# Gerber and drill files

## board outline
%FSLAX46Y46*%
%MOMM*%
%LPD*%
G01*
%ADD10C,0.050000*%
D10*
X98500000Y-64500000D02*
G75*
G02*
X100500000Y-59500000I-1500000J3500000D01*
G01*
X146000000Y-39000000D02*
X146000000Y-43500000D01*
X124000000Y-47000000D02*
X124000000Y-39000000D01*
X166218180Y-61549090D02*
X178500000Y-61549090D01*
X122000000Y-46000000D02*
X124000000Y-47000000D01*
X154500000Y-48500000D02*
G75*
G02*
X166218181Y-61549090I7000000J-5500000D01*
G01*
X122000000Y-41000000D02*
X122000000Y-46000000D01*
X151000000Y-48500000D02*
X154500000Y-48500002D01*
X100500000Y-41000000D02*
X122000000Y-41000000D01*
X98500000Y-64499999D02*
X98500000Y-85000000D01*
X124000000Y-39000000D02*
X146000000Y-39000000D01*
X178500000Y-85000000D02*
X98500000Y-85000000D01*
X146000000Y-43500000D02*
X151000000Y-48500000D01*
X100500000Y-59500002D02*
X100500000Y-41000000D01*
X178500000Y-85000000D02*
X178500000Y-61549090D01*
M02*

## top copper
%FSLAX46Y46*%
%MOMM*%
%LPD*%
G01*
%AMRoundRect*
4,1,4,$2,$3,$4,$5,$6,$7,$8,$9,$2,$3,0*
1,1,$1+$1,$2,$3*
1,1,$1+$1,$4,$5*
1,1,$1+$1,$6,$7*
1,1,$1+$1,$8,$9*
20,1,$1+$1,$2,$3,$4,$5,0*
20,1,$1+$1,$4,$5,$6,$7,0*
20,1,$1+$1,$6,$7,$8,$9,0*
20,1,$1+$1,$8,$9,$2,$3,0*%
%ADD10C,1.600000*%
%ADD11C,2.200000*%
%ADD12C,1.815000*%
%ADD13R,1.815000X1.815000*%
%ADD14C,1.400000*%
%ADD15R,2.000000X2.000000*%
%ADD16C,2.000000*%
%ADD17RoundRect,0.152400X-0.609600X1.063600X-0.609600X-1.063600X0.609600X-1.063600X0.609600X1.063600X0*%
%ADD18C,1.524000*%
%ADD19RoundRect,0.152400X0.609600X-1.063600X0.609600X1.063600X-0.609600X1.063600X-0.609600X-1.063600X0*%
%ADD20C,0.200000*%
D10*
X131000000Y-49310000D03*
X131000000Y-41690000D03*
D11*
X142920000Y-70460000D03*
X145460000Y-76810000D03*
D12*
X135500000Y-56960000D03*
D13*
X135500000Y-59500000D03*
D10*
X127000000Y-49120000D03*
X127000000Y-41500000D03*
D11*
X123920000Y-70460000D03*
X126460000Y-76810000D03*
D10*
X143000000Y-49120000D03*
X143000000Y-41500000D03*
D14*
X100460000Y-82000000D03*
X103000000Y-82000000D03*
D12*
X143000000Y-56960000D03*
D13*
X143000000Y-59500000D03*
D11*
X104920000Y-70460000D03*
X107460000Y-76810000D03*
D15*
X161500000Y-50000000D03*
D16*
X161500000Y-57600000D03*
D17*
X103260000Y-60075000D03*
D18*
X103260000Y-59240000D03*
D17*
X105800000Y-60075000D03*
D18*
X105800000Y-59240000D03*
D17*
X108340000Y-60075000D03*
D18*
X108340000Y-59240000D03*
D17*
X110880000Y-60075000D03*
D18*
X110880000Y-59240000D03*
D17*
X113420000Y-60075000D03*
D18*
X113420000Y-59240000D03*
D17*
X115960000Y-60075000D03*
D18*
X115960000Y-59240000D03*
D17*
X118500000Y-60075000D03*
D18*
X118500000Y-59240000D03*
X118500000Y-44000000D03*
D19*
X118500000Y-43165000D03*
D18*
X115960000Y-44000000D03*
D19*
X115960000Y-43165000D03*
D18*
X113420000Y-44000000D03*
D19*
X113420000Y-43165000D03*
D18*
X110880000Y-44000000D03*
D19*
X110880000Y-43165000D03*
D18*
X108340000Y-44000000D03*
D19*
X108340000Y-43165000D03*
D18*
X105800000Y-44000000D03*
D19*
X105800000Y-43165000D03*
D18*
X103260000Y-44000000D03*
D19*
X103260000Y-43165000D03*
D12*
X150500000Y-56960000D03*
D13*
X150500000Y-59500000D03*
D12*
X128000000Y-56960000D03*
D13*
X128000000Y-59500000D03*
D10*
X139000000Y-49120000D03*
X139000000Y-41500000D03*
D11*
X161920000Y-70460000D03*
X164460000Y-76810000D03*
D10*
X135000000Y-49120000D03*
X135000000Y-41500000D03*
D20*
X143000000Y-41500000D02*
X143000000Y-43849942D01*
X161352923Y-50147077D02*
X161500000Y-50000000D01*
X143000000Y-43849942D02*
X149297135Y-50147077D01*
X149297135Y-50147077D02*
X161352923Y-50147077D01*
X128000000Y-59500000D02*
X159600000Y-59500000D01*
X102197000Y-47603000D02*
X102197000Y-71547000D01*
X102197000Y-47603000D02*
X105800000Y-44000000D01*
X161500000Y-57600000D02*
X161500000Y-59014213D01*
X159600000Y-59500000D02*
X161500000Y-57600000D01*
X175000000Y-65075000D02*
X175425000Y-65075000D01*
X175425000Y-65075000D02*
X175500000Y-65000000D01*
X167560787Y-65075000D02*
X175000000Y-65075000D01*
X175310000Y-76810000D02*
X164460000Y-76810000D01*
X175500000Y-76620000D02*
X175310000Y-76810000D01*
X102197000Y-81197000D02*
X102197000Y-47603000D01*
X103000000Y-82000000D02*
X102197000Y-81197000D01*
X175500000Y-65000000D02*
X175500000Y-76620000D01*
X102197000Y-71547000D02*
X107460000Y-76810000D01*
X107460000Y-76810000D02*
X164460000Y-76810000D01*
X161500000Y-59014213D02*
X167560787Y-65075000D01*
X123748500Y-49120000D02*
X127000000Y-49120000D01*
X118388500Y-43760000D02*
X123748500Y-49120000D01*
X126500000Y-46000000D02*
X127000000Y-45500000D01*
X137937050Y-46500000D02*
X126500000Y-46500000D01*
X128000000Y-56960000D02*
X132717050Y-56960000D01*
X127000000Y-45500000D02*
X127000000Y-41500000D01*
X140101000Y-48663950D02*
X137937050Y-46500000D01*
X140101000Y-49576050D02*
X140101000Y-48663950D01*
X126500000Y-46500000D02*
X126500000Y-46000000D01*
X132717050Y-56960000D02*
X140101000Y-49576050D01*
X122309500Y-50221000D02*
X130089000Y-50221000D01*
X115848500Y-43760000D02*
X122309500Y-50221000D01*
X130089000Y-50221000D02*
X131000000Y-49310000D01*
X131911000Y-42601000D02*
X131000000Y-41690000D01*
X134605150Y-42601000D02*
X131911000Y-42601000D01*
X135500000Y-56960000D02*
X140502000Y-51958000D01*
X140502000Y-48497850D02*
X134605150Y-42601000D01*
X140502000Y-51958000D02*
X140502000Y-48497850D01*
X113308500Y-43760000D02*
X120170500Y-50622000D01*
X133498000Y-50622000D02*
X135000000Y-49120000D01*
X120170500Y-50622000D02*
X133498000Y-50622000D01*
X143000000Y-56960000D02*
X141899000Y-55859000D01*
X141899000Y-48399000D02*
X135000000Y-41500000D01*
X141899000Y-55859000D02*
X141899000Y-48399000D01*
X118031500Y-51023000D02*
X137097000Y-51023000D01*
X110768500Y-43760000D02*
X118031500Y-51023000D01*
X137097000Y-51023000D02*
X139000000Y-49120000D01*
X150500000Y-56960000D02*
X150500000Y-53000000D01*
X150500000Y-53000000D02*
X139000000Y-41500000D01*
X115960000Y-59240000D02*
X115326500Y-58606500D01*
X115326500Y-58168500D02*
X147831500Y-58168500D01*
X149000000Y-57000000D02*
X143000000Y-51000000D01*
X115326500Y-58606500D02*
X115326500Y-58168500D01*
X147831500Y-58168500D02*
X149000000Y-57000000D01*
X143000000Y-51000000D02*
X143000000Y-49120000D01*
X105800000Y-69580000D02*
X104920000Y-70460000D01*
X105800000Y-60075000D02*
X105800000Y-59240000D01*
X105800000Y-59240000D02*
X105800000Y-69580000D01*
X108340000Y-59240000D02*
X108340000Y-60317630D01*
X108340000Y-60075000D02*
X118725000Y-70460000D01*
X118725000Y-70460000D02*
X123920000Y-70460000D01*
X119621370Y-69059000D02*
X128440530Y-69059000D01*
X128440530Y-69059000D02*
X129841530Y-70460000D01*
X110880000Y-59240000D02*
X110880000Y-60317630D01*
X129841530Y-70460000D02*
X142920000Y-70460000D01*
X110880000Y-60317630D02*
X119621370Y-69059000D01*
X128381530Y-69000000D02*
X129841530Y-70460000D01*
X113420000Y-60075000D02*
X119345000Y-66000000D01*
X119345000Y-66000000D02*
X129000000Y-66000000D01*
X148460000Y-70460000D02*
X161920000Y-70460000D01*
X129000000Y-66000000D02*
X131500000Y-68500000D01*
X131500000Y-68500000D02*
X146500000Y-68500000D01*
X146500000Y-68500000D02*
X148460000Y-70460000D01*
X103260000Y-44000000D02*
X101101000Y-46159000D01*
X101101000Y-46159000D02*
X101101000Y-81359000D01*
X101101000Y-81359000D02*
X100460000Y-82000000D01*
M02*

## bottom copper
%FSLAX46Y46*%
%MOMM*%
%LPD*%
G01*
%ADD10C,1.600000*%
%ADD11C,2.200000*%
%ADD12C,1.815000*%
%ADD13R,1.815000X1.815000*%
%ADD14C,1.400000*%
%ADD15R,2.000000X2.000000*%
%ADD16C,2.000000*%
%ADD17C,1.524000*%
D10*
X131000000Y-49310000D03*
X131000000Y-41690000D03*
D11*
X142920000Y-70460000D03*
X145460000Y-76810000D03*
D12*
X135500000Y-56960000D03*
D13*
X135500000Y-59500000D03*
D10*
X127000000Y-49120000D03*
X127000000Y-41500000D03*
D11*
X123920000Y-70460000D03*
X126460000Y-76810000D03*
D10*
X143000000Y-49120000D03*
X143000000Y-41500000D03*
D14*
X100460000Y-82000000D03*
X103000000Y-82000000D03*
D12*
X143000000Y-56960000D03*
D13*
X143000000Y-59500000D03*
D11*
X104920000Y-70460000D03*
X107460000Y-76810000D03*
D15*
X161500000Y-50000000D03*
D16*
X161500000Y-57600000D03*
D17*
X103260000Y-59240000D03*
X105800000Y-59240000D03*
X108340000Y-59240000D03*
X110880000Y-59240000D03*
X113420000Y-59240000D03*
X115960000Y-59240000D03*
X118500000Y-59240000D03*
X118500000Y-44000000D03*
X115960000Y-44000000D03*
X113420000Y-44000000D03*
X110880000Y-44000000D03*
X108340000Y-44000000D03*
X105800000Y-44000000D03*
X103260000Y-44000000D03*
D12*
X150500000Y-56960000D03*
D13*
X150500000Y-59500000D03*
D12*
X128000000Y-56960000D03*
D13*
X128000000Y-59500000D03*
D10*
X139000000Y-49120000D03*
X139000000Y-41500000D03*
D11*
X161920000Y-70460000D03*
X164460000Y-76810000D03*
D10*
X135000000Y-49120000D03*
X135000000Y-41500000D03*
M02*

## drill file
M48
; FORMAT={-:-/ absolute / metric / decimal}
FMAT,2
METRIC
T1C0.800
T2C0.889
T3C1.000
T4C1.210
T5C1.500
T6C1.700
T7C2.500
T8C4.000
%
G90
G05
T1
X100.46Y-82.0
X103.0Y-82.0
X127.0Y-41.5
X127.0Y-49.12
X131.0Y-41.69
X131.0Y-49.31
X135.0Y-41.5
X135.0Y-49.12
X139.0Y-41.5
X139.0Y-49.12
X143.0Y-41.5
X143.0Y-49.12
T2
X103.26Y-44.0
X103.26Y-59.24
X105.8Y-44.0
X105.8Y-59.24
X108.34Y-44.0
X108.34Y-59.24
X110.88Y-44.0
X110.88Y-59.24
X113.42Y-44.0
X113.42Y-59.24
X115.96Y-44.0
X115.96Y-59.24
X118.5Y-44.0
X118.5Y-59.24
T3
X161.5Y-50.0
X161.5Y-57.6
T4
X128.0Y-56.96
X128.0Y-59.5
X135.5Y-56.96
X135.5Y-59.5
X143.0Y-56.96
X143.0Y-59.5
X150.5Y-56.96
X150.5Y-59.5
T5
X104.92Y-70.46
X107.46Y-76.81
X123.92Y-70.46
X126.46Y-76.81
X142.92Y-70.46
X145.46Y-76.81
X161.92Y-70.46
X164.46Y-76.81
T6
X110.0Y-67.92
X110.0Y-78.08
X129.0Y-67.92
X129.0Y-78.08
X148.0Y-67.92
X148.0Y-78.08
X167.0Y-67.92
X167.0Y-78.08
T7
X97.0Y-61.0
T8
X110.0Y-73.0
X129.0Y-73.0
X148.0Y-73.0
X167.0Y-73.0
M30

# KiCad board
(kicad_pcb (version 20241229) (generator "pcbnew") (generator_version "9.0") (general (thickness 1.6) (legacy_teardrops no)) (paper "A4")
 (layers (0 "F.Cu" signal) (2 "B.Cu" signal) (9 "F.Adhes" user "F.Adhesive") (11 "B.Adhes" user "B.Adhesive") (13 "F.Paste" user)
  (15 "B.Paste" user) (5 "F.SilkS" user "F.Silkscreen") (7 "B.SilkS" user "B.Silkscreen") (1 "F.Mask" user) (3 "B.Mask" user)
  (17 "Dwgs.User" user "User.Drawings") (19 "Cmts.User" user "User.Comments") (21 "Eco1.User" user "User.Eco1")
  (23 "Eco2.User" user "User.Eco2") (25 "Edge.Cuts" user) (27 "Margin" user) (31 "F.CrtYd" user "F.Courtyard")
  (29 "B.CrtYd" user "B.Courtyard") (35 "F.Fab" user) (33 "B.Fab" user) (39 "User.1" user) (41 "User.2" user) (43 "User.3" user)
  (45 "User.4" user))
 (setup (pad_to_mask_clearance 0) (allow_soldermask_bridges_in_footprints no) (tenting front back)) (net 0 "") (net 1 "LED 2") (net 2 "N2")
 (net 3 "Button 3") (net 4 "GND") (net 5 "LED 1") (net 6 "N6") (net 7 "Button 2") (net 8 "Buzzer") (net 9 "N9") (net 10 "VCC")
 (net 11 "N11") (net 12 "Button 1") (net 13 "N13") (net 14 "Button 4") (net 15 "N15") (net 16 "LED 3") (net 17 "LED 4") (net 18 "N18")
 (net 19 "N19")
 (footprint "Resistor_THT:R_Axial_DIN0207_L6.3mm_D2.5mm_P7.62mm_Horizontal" (layer "F.Cu") (at 131 49.31 90)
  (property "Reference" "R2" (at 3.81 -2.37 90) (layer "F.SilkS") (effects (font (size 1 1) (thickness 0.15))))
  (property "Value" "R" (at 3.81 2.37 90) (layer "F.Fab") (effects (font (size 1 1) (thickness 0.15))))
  (pad "1" thru_hole circle (at 0 0 90) (size 1.6 1.6) (drill 0.8) (layers "*.Cu" "*.Mask") (remove_unused_layers no) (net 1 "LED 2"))
  (pad "2" thru_hole circle (at 7.62 0 90) (size 1.6 1.6) (drill 0.8) (layers "*.Cu" "*.Mask") (remove_unused_layers no) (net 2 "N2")))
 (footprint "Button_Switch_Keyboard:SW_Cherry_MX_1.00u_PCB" (layer "F.Cu") (at 142.92 70.46 90)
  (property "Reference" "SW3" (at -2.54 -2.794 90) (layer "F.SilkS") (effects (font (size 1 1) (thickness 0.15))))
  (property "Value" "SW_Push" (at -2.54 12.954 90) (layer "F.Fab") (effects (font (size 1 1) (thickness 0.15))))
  (pad "" np_thru_hole circle (at -7.62 5.08 90) (size 1.7 1.7) (drill 1.7) (layers "*.Cu" "*.Mask"))
  (pad "" np_thru_hole circle (at -2.54 5.08 90) (size 4 4) (drill 4) (layers "*.Cu" "*.Mask"))
  (pad "" np_thru_hole circle (at 2.54 5.08 90) (size 1.7 1.7) (drill 1.7) (layers "*.Cu" "*.Mask"))
  (pad "1" thru_hole circle (at 0 0 90) (size 2.2 2.2) (drill 1.5) (layers "*.Cu" "*.Mask") (remove_unused_layers no) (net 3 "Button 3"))
  (pad "2" thru_hole circle (at -6.35 2.54 90) (size 2.2 2.2) (drill 1.5) (layers "*.Cu" "*.Mask") (remove_unused_layers no) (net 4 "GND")))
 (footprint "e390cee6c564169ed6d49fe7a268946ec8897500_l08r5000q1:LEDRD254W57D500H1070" (layer "F.Cu") (at 135.5 58.23 90)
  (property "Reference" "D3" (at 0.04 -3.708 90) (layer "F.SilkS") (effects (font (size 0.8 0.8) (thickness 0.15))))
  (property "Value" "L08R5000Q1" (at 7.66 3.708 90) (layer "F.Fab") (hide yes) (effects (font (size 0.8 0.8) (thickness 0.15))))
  (pad "A" thru_hole circle (at 1.27 0 90) (size 1.815 1.815) (drill 1.21) (layers "*.Cu" "*.Mask") (remove_unused_layers no) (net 2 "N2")
   (solder_mask_margin 0.102))
  (pad "C" thru_hole rect (at -1.27 0 90) (size 1.815 1.815) (drill 1.21) (layers "*.Cu" "*.Mask") (remove_unused_layers no) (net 4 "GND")
   (solder_mask_margin 0.102)))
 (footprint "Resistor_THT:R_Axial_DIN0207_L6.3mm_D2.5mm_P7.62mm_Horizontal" (layer "F.Cu") (at 127 49.12 90)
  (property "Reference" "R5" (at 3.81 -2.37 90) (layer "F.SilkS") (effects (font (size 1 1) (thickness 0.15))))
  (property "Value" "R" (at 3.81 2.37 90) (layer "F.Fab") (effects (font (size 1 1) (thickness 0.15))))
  (pad "1" thru_hole circle (at 0 0 90) (size 1.6 1.6) (drill 0.8) (layers "*.Cu" "*.Mask") (remove_unused_layers no) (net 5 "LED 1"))
  (pad "2" thru_hole circle (at 7.62 0 90) (size 1.6 1.6) (drill 0.8) (layers "*.Cu" "*.Mask") (remove_unused_layers no) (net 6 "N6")))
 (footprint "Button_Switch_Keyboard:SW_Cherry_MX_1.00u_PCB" (layer "F.Cu") (at 123.92 70.46 90)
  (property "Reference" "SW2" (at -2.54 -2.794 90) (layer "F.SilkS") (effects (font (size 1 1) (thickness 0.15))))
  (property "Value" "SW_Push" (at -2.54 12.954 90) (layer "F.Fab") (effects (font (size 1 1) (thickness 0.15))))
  (pad "" np_thru_hole circle (at -7.62 5.08 90) (size 1.7 1.7) (drill 1.7) (layers "*.Cu" "*.Mask"))
  (pad "" np_thru_hole circle (at -2.54 5.08 90) (size 4 4) (drill 4) (layers "*.Cu" "*.Mask"))
  (pad "" np_thru_hole circle (at 2.54 5.08 90) (size 1.7 1.7) (drill 1.7) (layers "*.Cu" "*.Mask"))
  (pad "1" thru_hole circle (at 0 0 90) (size 2.2 2.2) (drill 1.5) (layers "*.Cu" "*.Mask") (remove_unused_layers no) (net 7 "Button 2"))
  (pad "2" thru_hole circle (at -6.35 2.54 90) (size 2.2 2.2) (drill 1.5) (layers "*.Cu" "*.Mask") (remove_unused_layers no) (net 4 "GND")))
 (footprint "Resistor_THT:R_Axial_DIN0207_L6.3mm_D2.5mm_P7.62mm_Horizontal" (layer "F.Cu") (at 143 49.12 90)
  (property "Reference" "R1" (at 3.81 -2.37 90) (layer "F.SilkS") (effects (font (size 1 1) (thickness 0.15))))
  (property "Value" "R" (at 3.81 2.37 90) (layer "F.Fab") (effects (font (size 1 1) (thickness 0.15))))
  (pad "1" thru_hole circle (at 0 0 90) (size 1.6 1.6) (drill 0.8) (layers "*.Cu" "*.Mask") (remove_unused_layers no) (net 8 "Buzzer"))
  (pad "2" thru_hole circle (at 7.62 0 90) (size 1.6 1.6) (drill 0.8) (layers "*.Cu" "*.Mask") (remove_unused_layers no) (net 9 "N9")))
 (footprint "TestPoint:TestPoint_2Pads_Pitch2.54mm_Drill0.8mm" (layer "F.Cu") (at 100.46 82)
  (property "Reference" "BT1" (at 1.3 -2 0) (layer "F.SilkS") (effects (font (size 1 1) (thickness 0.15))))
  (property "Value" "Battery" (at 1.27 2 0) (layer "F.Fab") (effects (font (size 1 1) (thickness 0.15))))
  (pad "1" thru_hole circle (at 0 0) (size 1.4 1.4) (drill 0.8) (layers "*.Cu" "*.Mask") (remove_unused_layers no) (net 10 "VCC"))
  (pad "2" thru_hole circle (at 2.54 0) (size 1.4 1.4) (drill 0.8) (layers "*.Cu" "*.Mask") (remove_unused_layers no) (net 4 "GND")))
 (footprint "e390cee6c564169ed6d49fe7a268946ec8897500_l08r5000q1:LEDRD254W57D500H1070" (layer "F.Cu") (at 143 58.23 90)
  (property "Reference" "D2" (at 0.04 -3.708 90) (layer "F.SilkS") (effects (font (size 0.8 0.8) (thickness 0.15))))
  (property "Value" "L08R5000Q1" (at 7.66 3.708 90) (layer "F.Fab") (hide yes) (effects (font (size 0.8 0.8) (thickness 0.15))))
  (pad "A" thru_hole circle (at 1.27 0 90) (size 1.815 1.815) (drill 1.21) (layers "*.Cu" "*.Mask") (remove_unused_layers no) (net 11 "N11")
   (solder_mask_margin 0.102))
  (pad "C" thru_hole rect (at -1.27 0 90) (size 1.815 1.815) (drill 1.21) (layers "*.Cu" "*.Mask") (remove_unused_layers no) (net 4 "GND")
   (solder_mask_margin 0.102)))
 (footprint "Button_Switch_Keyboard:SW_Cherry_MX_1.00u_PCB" (layer "F.Cu") (at 104.92 70.46 90)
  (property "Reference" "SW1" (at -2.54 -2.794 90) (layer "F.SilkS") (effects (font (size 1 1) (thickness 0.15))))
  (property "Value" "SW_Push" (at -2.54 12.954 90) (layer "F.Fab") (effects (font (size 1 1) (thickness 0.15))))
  (pad "" np_thru_hole circle (at -7.62 5.08 90) (size 1.7 1.7) (drill 1.7) (layers "*.Cu" "*.Mask"))
  (pad "" np_thru_hole circle (at -2.54 5.08 90) (size 4 4) (drill 4) (layers "*.Cu" "*.Mask"))
  (pad "" np_thru_hole circle (at 2.54 5.08 90) (size 1.7 1.7) (drill 1.7) (layers "*.Cu" "*.Mask"))
  (pad "1" thru_hole circle (at 0 0 90) (size 2.2 2.2) (drill 1.5) (layers "*.Cu" "*.Mask") (remove_unused_layers no) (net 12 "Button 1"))
  (pad "2" thru_hole circle (at -6.35 2.54 90) (size 2.2 2.2) (drill 1.5) (layers "*.Cu" "*.Mask") (remove_unused_layers no) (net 4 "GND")))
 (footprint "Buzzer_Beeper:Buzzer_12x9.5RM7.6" (layer "F.Cu") (at 161.5 50 -90)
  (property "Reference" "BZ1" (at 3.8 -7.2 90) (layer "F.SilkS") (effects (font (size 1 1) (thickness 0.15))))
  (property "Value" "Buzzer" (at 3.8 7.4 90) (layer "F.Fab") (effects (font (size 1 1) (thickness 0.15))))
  (pad "1" thru_hole rect (at 0 0 270) (size 2 2) (drill 1) (layers "*.Cu" "*.Mask") (remove_unused_layers no) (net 9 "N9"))
  (pad "2" thru_hole circle (at 7.6 0 270) (size 2 2) (drill 1) (layers "*.Cu" "*.Mask") (remove_unused_layers no) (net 4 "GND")))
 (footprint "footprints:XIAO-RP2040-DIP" (layer "F.Cu") (at 110.88 51.62 90)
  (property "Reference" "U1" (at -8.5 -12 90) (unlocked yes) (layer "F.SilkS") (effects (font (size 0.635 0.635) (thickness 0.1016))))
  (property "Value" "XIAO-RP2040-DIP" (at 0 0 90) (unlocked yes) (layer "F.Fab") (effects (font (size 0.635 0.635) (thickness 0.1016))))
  (pad "1" smd roundrect (at -8.455 -7.62 270) (size 2.432 1.524) (layers "F.Cu" "F.Mask") (roundrect_rratio 0.1) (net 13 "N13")
   (thermal_bridge_angle 45))
  (pad "1" thru_hole circle (at -7.62 -7.62 270) (size 1.524 1.524) (drill 0.889) (layers "*.Cu" "*.Mask") (remove_unused_layers no)
   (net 13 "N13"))
  (pad "2" smd roundrect (at -8.455 -5.08 270) (size 2.432 1.524) (layers "F.Cu" "F.Mask") (roundrect_rratio 0.1) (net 12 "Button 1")
   (thermal_bridge_angle 45))
  (pad "2" thru_hole circle (at -7.62 -5.08 270) (size 1.524 1.524) (drill 0.889) (layers "*.Cu" "*.Mask") (remove_unused_layers no)
   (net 12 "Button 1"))
  (pad "3" smd roundrect (at -8.455 -2.54 270) (size 2.432 1.524) (layers "F.Cu" "F.Mask") (roundrect_rratio 0.1) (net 7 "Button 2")
   (thermal_bridge_angle 45))
  (pad "3" thru_hole circle (at -7.62 -2.54 270) (size 1.524 1.524) (drill 0.889) (layers "*.Cu" "*.Mask") (remove_unused_layers no)
   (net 7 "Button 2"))
  (pad "4" smd roundrect (at -8.455 0 270) (size 2.432 1.524) (layers "F.Cu" "F.Mask") (roundrect_rratio 0.1) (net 3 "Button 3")
   (thermal_bridge_angle 45))
  (pad "4" thru_hole circle (at -7.62 0 270) (size 1.524 1.524) (drill 0.889) (layers "*.Cu" "*.Mask") (remove_unused_layers no)
   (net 3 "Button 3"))
  (pad "5" smd roundrect (at -8.455 2.54 270) (size 2.432 1.524) (layers "F.Cu" "F.Mask") (roundrect_rratio 0.1) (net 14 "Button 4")
   (thermal_bridge_angle 45))
  (pad "5" thru_hole circle (at -7.62 2.54 270) (size 1.524 1.524) (drill 0.889) (layers "*.Cu" "*.Mask") (remove_unused_layers no)
   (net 14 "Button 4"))
  (pad "6" smd roundrect (at -8.455 5.08 270) (size 2.432 1.524) (layers "F.Cu" "F.Mask") (roundrect_rratio 0.1) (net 8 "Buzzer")
   (thermal_bridge_angle 45))
  (pad "6" thru_hole circle (at -7.62 5.08 270) (size 1.524 1.524) (drill 0.889) (layers "*.Cu" "*.Mask") (remove_unused_layers no)
   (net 8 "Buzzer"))
  (pad "7" smd roundrect (at -8.455 7.62 270) (size 2.432 1.524) (layers "F.Cu" "F.Mask") (roundrect_rratio 0.1) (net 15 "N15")
   (thermal_bridge_angle 45))
  (pad "7" thru_hole circle (at -7.62 7.62 270) (size 1.524 1.524) (drill 0.889) (layers "*.Cu" "*.Mask") (remove_unused_layers no)
   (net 15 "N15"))
  (pad "8" thru_hole circle (at 7.62 7.62 90) (size 1.524 1.524) (drill 0.889) (layers "*.Cu" "*.Mask") (remove_unused_layers no)
   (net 5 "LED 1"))
  (pad "8" smd roundrect (at 8.455 7.62 90) (size 2.432 1.524) (layers "F.Cu" "F.Mask") (roundrect_rratio 0.1) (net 5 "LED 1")
   (thermal_bridge_angle 45))
  (pad "9" thru_hole circle (at 7.62 5.08 90) (size 1.524 1.524) (drill 0.889) (layers "*.Cu" "*.Mask") (remove_unused_layers no)
   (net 1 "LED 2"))
  (pad "9" smd roundrect (at 8.455 5.08 90) (size 2.432 1.524) (layers "F.Cu" "F.Mask") (roundrect_rratio 0.1) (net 1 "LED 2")
   (thermal_bridge_angle 45))
  (pad "10" thru_hole circle (at 7.62 2.54 90) (size 1.524 1.524) (drill 0.889) (layers "*.Cu" "*.Mask") (remove_unused_layers no)
   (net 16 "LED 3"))
  (pad "10" smd roundrect (at 8.455 2.54 90) (size 2.432 1.524) (layers "F.Cu" "F.Mask") (roundrect_rratio 0.1) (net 16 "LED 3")
   (thermal_bridge_angle 45))
  (pad "11" thru_hole circle (at 7.62 0 90) (size 1.524 1.524) (drill 0.889) (layers "*.Cu" "*.Mask") (remove_unused_layers no)
   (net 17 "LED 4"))
  (pad "11" smd roundrect (at 8.455 0 90) (size 2.432 1.524) (layers "F.Cu" "F.Mask") (roundrect_rratio 0.1) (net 17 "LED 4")
   (thermal_bridge_angle 45))
  (pad "12" thru_hole circle (at 7.62 -2.54 90) (size 1.524 1.524) (drill 0.889) (layers "*.Cu" "*.Mask") (remove_unused_layers no)
   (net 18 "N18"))
  (pad "12" smd roundrect (at 8.455 -2.54 90) (size 2.432 1.524) (layers "F.Cu" "F.Mask") (roundrect_rratio 0.1) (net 18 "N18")
   (thermal_bridge_angle 45))
  (pad "13" thru_hole circle (at 7.62 -5.08 90) (size 1.524 1.524) (drill 0.889) (layers "*.Cu" "*.Mask") (remove_unused_layers no)
   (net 4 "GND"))
  (pad "13" smd roundrect (at 8.455 -5.08 90) (size 2.432 1.524) (layers "F.Cu" "F.Mask") (roundrect_rratio 0.1) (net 4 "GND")
   (thermal_bridge_angle 45))
  (pad "14" thru_hole circle (at 7.62 -7.62 90) (size 1.524 1.524) (drill 0.889) (layers "*.Cu" "*.Mask") (remove_unused_layers no)
   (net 10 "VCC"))
  (pad "14" smd roundrect (at 8.455 -7.62 90) (size 2.432 1.524) (layers "F.Cu" "F.Mask") (roundrect_rratio 0.1) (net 10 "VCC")
   (thermal_bridge_angle 45)))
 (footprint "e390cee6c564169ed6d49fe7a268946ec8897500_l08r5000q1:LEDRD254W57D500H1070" (layer "F.Cu") (at 150.5 58.23 90)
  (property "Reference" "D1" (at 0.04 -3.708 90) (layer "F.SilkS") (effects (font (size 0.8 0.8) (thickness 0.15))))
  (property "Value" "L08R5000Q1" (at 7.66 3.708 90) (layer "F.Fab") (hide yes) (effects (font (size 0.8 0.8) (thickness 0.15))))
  (pad "A" thru_hole circle (at 1.27 0 90) (size 1.815 1.815) (drill 1.21) (layers "*.Cu" "*.Mask") (remove_unused_layers no) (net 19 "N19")
   (solder_mask_margin 0.102))
  (pad "C" thru_hole rect (at -1.27 0 90) (size 1.815 1.815) (drill 1.21) (layers "*.Cu" "*.Mask") (remove_unused_layers no) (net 4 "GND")
   (solder_mask_margin 0.102)))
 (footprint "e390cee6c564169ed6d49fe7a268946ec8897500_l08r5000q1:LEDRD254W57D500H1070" (layer "F.Cu") (at 128 58.23 90)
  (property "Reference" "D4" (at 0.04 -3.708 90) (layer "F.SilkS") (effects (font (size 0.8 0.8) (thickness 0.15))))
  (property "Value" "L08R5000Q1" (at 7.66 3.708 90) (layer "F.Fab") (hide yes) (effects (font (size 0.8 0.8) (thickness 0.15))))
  (pad "A" thru_hole circle (at 1.27 0 90) (size 1.815 1.815) (drill 1.21) (layers "*.Cu" "*.Mask") (remove_unused_layers no) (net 6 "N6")
   (solder_mask_margin 0.102))
  (pad "C" thru_hole rect (at -1.27 0 90) (size 1.815 1.815) (drill 1.21) (layers "*.Cu" "*.Mask") (remove_unused_layers no) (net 4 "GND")
   (solder_mask_margin 0.102)))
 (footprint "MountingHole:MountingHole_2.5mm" (layer "F.Cu") (at 97 61)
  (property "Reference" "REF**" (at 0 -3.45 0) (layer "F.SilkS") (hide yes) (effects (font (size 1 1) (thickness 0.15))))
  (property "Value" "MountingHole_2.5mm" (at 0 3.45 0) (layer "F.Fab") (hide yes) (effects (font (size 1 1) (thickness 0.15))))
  (pad "" np_thru_hole circle (at 0 0) (size 2.5 2.5) (drill 2.5) (layers "*.Cu" "*.Mask")))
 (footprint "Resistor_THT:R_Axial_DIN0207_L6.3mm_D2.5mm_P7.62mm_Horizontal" (layer "F.Cu") (at 139 49.12 90)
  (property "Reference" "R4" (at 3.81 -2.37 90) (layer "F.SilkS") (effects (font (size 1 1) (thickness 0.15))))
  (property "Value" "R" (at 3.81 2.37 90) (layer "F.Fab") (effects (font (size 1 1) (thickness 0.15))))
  (pad "1" thru_hole circle (at 0 0 90) (size 1.6 1.6) (drill 0.8) (layers "*.Cu" "*.Mask") (remove_unused_layers no) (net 17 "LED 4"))
  (pad "2" thru_hole circle (at 7.62 0 90) (size 1.6 1.6) (drill 0.8) (layers "*.Cu" "*.Mask") (remove_unused_layers no) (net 19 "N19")))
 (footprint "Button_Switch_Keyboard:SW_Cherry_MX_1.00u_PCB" (layer "F.Cu") (at 161.92 70.46 90)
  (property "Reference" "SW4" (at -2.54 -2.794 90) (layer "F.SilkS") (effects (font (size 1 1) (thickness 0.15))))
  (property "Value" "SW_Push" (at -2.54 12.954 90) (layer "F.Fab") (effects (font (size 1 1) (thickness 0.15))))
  (pad "" np_thru_hole circle (at -7.62 5.08 90) (size 1.7 1.7) (drill 1.7) (layers "*.Cu" "*.Mask"))
  (pad "" np_thru_hole circle (at -2.54 5.08 90) (size 4 4) (drill 4) (layers "*.Cu" "*.Mask"))
  (pad "" np_thru_hole circle (at 2.54 5.08 90) (size 1.7 1.7) (drill 1.7) (layers "*.Cu" "*.Mask"))
  (pad "1" thru_hole circle (at 0 0 90) (size 2.2 2.2) (drill 1.5) (layers "*.Cu" "*.Mask") (remove_unused_layers no) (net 14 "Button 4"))
  (pad "2" thru_hole circle (at -6.35 2.54 90) (size 2.2 2.2) (drill 1.5) (layers "*.Cu" "*.Mask") (remove_unused_layers no) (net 4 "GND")))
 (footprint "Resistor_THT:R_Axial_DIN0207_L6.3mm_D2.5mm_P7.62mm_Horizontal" (layer "F.Cu") (at 135 49.12 90)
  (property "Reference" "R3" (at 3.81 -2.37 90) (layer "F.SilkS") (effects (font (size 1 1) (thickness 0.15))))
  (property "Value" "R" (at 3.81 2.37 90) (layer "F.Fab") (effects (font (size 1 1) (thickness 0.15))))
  (pad "1" thru_hole circle (at 0 0 90) (size 1.6 1.6) (drill 0.8) (layers "*.Cu" "*.Mask") (remove_unused_layers no) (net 16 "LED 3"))
  (pad "2" thru_hole circle (at 7.62 0 90) (size 1.6 1.6) (drill 0.8) (layers "*.Cu" "*.Mask") (remove_unused_layers no) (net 11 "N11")))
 (gr_arc (start 98.5 64.5) (mid 93.464466 59.585786) (end 100.5 59.5) (stroke (width 0.05) (type default)) (layer "Edge.Cuts"))
 (gr_line (start 146 39) (end 146 43.5) (stroke (width 0.05) (type default)) (layer "Edge.Cuts"))
 (gr_line (start 124 47) (end 124 39) (stroke (width 0.05) (type default)) (layer "Edge.Cuts"))
 (gr_line (start 166.21818 61.54909) (end 178.5 61.54909) (stroke (width 0.05) (type default)) (layer "Edge.Cuts"))
 (gr_line (start 122 46) (end 124 47) (stroke (width 0.05) (type default)) (layer "Edge.Cuts"))
 (gr_arc (start 154.5 48.5) (mid 168.123546 48.052006) (end 166.218181 61.54909) (stroke (width 0.05) (type default)) (layer "Edge.Cuts"))
 (gr_line (start 122 41) (end 122 46) (stroke (width 0.05) (type default)) (layer "Edge.Cuts"))
 (gr_line (start 151 48.5) (end 154.5 48.500002) (stroke (width 0.05) (type default)) (layer "Edge.Cuts"))
 (gr_line (start 100.5 41) (end 122 41) (stroke (width 0.05) (type default)) (layer "Edge.Cuts"))
 (gr_line (start 98.5 64.499999) (end 98.5 85) (stroke (width 0.05) (type default)) (layer "Edge.Cuts"))
 (gr_line (start 124 39) (end 146 39) (stroke (width 0.05) (type default)) (layer "Edge.Cuts"))
 (gr_line (start 178.5 85) (end 98.5 85) (stroke (width 0.05) (type default)) (layer "Edge.Cuts"))
 (gr_line (start 146 43.5) (end 151 48.5) (stroke (width 0.05) (type default)) (layer "Edge.Cuts"))
 (gr_line (start 100.5 59.500002) (end 100.5 41) (stroke (width 0.05) (type default)) (layer "Edge.Cuts"))
 (gr_line (start 178.5 85) (end 178.5 61.54909) (stroke (width 0.05) (type default)) (layer "Edge.Cuts"))
 (segment (start 143 41.5) (end 143 43.849942) (width 0.2) (layer "F.Cu") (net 9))
 (segment (start 161.352923 50.147077) (end 161.5 50) (width 0.2) (layer "F.Cu") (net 9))
 (segment (start 143 43.849942) (end 149.297135 50.147077) (width 0.2) (layer "F.Cu") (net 9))
 (segment (start 149.297135 50.147077) (end 161.352923 50.147077) (width 0.2) (layer "F.Cu") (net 9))
 (segment (start 128 59.5) (end 159.6 59.5) (width 0.2) (layer "F.Cu") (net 4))
 (segment (start 102.197 47.603) (end 102.197 71.547) (width 0.2) (layer "F.Cu") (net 4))
 (segment (start 102.197 47.603) (end 105.8 44) (width 0.2) (layer "F.Cu") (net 4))
 (segment (start 161.5 57.6) (end 161.5 59.014213) (width 0.2) (layer "F.Cu") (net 4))
 (segment (start 159.6 59.5) (end 161.5 57.6) (width 0.2) (layer "F.Cu") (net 4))
 (segment (start 175 65.075) (end 175.425 65.075) (width 0.2) (layer "F.Cu") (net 4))
 (segment (start 175.425 65.075) (end 175.5 65) (width 0.2) (layer "F.Cu") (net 4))
 (segment (start 167.560787 65.075) (end 175 65.075) (width 0.2) (layer "F.Cu") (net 4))
 (segment (start 175.31 76.81) (end 164.46 76.81) (width 0.2) (layer "F.Cu") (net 4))
 (segment (start 175.5 76.62) (end 175.31 76.81) (width 0.2) (layer "F.Cu") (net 4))
 (segment (start 102.197 81.197) (end 102.197 47.603) (width 0.2) (layer "F.Cu") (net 4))
 (segment (start 103 82) (end 102.197 81.197) (width 0.2) (layer "F.Cu") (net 4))
 (segment (start 175.5 65) (end 175.5 76.62) (width 0.2) (layer "F.Cu") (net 4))
 (segment (start 102.197 71.547) (end 107.46 76.81) (width 0.2) (layer "F.Cu") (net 4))
 (segment (start 107.46 76.81) (end 164.46 76.81) (width 0.2) (layer "F.Cu") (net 4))
 (segment (start 161.5 59.014213) (end 167.560787 65.075) (width 0.2) (layer "F.Cu") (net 4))
 (segment (start 123.7485 49.12) (end 127 49.12) (width 0.2) (layer "F.Cu") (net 5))
 (segment (start 118.3885 43.76) (end 123.7485 49.12) (width 0.2) (layer "F.Cu") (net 5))
 (segment (start 126.5 46) (end 127 45.5) (width 0.2) (layer "F.Cu") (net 6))
 (segment (start 137.93705 46.5) (end 126.5 46.5) (width 0.2) (layer "F.Cu") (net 6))
 (segment (start 128 56.96) (end 132.71705 56.96) (width 0.2) (layer "F.Cu") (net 6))
 (segment (start 127 45.5) (end 127 41.5) (width 0.2) (layer "F.Cu") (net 6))
 (segment (start 140.101 48.66395) (end 137.93705 46.5) (width 0.2) (layer "F.Cu") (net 6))
 (segment (start 140.101 49.57605) (end 140.101 48.66395) (width 0.2) (layer "F.Cu") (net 6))
 (segment (start 126.5 46.5) (end 126.5 46) (width 0.2) (layer "F.Cu") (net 6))
 (segment (start 132.71705 56.96) (end 140.101 49.57605) (width 0.2) (layer "F.Cu") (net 6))
 (segment (start 122.3095 50.221) (end 130.089 50.221) (width 0.2) (layer "F.Cu") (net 1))
 (segment (start 115.8485 43.76) (end 122.3095 50.221) (width 0.2) (layer "F.Cu") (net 1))
 (segment (start 130.089 50.221) (end 131 49.31) (width 0.2) (layer "F.Cu") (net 1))
 (segment (start 131.911 42.601) (end 131 41.69) (width 0.2) (layer "F.Cu") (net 2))
 (segment (start 134.60515 42.601) (end 131.911 42.601) (width 0.2) (layer "F.Cu") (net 2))
 (segment (start 135.5 56.96) (end 140.502 51.958) (width 0.2) (layer "F.Cu") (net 2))
 (segment (start 140.502 48.49785) (end 134.60515 42.601) (width 0.2) (layer "F.Cu") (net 2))
 (segment (start 140.502 51.958) (end 140.502 48.49785) (width 0.2) (layer "F.Cu") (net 2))
 (segment (start 113.3085 43.76) (end 120.1705 50.622) (width 0.2) (layer "F.Cu") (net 16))
 (segment (start 133.498 50.622) (end 135 49.12) (width 0.2) (layer "F.Cu") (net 16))
 (segment (start 120.1705 50.622) (end 133.498 50.622) (width 0.2) (layer "F.Cu") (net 16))
 (segment (start 143 56.96) (end 141.899 55.859) (width 0.2) (layer "F.Cu") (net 11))
 (segment (start 141.899 48.399) (end 135 41.5) (width 0.2) (layer "F.Cu") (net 11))
 (segment (start 141.899 55.859) (end 141.899 48.399) (width 0.2) (layer "F.Cu") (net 11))
 (segment (start 118.0315 51.023) (end 137.097 51.023) (width 0.2) (layer "F.Cu") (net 17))
 (segment (start 110.7685 43.76) (end 118.0315 51.023) (width 0.2) (layer "F.Cu") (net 17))
 (segment (start 137.097 51.023) (end 139 49.12) (width 0.2) (layer "F.Cu") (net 17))
 (segment (start 150.5 56.96) (end 150.5 53) (width 0.2) (layer "F.Cu") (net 19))
 (segment (start 150.5 53) (end 139 41.5) (width 0.2) (layer "F.Cu") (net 19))
 (segment (start 115.96 59.24) (end 115.3265 58.6065) (width 0.2) (layer "F.Cu") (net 8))
 (segment (start 115.3265 58.1685) (end 147.8315 58.1685) (width 0.2) (layer "F.Cu") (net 8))
 (segment (start 149 57) (end 143 51) (width 0.2) (layer "F.Cu") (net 8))
 (segment (start 115.3265 58.6065) (end 115.3265 58.1685) (width 0.2) (layer "F.Cu") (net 8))
 (segment (start 147.8315 58.1685) (end 149 57) (width 0.2) (layer "F.Cu") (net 8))
 (segment (start 143 51) (end 143 49.12) (width 0.2) (layer "F.Cu") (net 8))
 (segment (start 105.8 69.58) (end 104.92 70.46) (width 0.2) (layer "F.Cu") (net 12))
 (segment (start 105.8 60.075) (end 105.8 59.24) (width 0.2) (layer "F.Cu") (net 12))
 (segment (start 105.8 59.24) (end 105.8 69.58) (width 0.2) (layer "F.Cu") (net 12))
 (segment (start 108.34 59.24) (end 108.34 60.31763) (width 0.2) (layer "F.Cu") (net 7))
 (segment (start 108.34 60.075) (end 118.725 70.46) (width 0.2) (layer "F.Cu") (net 7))
 (segment (start 118.725 70.46) (end 123.92 70.46) (width 0.2) (layer "F.Cu") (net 7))
 (segment (start 119.62137 69.059) (end 128.44053 69.059) (width 0.2) (layer "F.Cu") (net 3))
 (segment (start 128.44053 69.059) (end 129.84153 70.46) (width 0.2) (layer "F.Cu") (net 3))
 (segment (start 110.88 59.24) (end 110.88 60.31763) (width 0.2) (layer "F.Cu") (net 3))
 (segment (start 129.84153 70.46) (end 142.92 70.46) (width 0.2) (layer "F.Cu") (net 3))
 (segment (start 110.88 60.31763) (end 119.62137 69.059) (width 0.2) (layer "F.Cu") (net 3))
 (segment (start 128.38153 69) (end 129.84153 70.46) (width 0.2) (layer "F.Cu") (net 3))
 (segment (start 113.42 60.075) (end 119.345 66) (width 0.2) (layer "F.Cu") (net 14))
 (segment (start 119.345 66) (end 129 66) (width 0.2) (layer "F.Cu") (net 14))
 (segment (start 148.46 70.46) (end 161.92 70.46) (width 0.2) (layer "F.Cu") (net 14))
 (segment (start 129 66) (end 131.5 68.5) (width 0.2) (layer "F.Cu") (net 14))
 (segment (start 131.5 68.5) (end 146.5 68.5) (width 0.2) (layer "F.Cu") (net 14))
 (segment (start 146.5 68.5) (end 148.46 70.46) (width 0.2) (layer "F.Cu") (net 14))
 (segment (start 103.26 44) (end 101.101 46.159) (width 0.2) (layer "F.Cu") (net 10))
 (segment (start 101.101 46.159) (end 101.101 81.359) (width 0.2) (layer "F.Cu") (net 10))
 (segment (start 101.101 81.359) (end 100.46 82) (width 0.2) (layer "F.Cu") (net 10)))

